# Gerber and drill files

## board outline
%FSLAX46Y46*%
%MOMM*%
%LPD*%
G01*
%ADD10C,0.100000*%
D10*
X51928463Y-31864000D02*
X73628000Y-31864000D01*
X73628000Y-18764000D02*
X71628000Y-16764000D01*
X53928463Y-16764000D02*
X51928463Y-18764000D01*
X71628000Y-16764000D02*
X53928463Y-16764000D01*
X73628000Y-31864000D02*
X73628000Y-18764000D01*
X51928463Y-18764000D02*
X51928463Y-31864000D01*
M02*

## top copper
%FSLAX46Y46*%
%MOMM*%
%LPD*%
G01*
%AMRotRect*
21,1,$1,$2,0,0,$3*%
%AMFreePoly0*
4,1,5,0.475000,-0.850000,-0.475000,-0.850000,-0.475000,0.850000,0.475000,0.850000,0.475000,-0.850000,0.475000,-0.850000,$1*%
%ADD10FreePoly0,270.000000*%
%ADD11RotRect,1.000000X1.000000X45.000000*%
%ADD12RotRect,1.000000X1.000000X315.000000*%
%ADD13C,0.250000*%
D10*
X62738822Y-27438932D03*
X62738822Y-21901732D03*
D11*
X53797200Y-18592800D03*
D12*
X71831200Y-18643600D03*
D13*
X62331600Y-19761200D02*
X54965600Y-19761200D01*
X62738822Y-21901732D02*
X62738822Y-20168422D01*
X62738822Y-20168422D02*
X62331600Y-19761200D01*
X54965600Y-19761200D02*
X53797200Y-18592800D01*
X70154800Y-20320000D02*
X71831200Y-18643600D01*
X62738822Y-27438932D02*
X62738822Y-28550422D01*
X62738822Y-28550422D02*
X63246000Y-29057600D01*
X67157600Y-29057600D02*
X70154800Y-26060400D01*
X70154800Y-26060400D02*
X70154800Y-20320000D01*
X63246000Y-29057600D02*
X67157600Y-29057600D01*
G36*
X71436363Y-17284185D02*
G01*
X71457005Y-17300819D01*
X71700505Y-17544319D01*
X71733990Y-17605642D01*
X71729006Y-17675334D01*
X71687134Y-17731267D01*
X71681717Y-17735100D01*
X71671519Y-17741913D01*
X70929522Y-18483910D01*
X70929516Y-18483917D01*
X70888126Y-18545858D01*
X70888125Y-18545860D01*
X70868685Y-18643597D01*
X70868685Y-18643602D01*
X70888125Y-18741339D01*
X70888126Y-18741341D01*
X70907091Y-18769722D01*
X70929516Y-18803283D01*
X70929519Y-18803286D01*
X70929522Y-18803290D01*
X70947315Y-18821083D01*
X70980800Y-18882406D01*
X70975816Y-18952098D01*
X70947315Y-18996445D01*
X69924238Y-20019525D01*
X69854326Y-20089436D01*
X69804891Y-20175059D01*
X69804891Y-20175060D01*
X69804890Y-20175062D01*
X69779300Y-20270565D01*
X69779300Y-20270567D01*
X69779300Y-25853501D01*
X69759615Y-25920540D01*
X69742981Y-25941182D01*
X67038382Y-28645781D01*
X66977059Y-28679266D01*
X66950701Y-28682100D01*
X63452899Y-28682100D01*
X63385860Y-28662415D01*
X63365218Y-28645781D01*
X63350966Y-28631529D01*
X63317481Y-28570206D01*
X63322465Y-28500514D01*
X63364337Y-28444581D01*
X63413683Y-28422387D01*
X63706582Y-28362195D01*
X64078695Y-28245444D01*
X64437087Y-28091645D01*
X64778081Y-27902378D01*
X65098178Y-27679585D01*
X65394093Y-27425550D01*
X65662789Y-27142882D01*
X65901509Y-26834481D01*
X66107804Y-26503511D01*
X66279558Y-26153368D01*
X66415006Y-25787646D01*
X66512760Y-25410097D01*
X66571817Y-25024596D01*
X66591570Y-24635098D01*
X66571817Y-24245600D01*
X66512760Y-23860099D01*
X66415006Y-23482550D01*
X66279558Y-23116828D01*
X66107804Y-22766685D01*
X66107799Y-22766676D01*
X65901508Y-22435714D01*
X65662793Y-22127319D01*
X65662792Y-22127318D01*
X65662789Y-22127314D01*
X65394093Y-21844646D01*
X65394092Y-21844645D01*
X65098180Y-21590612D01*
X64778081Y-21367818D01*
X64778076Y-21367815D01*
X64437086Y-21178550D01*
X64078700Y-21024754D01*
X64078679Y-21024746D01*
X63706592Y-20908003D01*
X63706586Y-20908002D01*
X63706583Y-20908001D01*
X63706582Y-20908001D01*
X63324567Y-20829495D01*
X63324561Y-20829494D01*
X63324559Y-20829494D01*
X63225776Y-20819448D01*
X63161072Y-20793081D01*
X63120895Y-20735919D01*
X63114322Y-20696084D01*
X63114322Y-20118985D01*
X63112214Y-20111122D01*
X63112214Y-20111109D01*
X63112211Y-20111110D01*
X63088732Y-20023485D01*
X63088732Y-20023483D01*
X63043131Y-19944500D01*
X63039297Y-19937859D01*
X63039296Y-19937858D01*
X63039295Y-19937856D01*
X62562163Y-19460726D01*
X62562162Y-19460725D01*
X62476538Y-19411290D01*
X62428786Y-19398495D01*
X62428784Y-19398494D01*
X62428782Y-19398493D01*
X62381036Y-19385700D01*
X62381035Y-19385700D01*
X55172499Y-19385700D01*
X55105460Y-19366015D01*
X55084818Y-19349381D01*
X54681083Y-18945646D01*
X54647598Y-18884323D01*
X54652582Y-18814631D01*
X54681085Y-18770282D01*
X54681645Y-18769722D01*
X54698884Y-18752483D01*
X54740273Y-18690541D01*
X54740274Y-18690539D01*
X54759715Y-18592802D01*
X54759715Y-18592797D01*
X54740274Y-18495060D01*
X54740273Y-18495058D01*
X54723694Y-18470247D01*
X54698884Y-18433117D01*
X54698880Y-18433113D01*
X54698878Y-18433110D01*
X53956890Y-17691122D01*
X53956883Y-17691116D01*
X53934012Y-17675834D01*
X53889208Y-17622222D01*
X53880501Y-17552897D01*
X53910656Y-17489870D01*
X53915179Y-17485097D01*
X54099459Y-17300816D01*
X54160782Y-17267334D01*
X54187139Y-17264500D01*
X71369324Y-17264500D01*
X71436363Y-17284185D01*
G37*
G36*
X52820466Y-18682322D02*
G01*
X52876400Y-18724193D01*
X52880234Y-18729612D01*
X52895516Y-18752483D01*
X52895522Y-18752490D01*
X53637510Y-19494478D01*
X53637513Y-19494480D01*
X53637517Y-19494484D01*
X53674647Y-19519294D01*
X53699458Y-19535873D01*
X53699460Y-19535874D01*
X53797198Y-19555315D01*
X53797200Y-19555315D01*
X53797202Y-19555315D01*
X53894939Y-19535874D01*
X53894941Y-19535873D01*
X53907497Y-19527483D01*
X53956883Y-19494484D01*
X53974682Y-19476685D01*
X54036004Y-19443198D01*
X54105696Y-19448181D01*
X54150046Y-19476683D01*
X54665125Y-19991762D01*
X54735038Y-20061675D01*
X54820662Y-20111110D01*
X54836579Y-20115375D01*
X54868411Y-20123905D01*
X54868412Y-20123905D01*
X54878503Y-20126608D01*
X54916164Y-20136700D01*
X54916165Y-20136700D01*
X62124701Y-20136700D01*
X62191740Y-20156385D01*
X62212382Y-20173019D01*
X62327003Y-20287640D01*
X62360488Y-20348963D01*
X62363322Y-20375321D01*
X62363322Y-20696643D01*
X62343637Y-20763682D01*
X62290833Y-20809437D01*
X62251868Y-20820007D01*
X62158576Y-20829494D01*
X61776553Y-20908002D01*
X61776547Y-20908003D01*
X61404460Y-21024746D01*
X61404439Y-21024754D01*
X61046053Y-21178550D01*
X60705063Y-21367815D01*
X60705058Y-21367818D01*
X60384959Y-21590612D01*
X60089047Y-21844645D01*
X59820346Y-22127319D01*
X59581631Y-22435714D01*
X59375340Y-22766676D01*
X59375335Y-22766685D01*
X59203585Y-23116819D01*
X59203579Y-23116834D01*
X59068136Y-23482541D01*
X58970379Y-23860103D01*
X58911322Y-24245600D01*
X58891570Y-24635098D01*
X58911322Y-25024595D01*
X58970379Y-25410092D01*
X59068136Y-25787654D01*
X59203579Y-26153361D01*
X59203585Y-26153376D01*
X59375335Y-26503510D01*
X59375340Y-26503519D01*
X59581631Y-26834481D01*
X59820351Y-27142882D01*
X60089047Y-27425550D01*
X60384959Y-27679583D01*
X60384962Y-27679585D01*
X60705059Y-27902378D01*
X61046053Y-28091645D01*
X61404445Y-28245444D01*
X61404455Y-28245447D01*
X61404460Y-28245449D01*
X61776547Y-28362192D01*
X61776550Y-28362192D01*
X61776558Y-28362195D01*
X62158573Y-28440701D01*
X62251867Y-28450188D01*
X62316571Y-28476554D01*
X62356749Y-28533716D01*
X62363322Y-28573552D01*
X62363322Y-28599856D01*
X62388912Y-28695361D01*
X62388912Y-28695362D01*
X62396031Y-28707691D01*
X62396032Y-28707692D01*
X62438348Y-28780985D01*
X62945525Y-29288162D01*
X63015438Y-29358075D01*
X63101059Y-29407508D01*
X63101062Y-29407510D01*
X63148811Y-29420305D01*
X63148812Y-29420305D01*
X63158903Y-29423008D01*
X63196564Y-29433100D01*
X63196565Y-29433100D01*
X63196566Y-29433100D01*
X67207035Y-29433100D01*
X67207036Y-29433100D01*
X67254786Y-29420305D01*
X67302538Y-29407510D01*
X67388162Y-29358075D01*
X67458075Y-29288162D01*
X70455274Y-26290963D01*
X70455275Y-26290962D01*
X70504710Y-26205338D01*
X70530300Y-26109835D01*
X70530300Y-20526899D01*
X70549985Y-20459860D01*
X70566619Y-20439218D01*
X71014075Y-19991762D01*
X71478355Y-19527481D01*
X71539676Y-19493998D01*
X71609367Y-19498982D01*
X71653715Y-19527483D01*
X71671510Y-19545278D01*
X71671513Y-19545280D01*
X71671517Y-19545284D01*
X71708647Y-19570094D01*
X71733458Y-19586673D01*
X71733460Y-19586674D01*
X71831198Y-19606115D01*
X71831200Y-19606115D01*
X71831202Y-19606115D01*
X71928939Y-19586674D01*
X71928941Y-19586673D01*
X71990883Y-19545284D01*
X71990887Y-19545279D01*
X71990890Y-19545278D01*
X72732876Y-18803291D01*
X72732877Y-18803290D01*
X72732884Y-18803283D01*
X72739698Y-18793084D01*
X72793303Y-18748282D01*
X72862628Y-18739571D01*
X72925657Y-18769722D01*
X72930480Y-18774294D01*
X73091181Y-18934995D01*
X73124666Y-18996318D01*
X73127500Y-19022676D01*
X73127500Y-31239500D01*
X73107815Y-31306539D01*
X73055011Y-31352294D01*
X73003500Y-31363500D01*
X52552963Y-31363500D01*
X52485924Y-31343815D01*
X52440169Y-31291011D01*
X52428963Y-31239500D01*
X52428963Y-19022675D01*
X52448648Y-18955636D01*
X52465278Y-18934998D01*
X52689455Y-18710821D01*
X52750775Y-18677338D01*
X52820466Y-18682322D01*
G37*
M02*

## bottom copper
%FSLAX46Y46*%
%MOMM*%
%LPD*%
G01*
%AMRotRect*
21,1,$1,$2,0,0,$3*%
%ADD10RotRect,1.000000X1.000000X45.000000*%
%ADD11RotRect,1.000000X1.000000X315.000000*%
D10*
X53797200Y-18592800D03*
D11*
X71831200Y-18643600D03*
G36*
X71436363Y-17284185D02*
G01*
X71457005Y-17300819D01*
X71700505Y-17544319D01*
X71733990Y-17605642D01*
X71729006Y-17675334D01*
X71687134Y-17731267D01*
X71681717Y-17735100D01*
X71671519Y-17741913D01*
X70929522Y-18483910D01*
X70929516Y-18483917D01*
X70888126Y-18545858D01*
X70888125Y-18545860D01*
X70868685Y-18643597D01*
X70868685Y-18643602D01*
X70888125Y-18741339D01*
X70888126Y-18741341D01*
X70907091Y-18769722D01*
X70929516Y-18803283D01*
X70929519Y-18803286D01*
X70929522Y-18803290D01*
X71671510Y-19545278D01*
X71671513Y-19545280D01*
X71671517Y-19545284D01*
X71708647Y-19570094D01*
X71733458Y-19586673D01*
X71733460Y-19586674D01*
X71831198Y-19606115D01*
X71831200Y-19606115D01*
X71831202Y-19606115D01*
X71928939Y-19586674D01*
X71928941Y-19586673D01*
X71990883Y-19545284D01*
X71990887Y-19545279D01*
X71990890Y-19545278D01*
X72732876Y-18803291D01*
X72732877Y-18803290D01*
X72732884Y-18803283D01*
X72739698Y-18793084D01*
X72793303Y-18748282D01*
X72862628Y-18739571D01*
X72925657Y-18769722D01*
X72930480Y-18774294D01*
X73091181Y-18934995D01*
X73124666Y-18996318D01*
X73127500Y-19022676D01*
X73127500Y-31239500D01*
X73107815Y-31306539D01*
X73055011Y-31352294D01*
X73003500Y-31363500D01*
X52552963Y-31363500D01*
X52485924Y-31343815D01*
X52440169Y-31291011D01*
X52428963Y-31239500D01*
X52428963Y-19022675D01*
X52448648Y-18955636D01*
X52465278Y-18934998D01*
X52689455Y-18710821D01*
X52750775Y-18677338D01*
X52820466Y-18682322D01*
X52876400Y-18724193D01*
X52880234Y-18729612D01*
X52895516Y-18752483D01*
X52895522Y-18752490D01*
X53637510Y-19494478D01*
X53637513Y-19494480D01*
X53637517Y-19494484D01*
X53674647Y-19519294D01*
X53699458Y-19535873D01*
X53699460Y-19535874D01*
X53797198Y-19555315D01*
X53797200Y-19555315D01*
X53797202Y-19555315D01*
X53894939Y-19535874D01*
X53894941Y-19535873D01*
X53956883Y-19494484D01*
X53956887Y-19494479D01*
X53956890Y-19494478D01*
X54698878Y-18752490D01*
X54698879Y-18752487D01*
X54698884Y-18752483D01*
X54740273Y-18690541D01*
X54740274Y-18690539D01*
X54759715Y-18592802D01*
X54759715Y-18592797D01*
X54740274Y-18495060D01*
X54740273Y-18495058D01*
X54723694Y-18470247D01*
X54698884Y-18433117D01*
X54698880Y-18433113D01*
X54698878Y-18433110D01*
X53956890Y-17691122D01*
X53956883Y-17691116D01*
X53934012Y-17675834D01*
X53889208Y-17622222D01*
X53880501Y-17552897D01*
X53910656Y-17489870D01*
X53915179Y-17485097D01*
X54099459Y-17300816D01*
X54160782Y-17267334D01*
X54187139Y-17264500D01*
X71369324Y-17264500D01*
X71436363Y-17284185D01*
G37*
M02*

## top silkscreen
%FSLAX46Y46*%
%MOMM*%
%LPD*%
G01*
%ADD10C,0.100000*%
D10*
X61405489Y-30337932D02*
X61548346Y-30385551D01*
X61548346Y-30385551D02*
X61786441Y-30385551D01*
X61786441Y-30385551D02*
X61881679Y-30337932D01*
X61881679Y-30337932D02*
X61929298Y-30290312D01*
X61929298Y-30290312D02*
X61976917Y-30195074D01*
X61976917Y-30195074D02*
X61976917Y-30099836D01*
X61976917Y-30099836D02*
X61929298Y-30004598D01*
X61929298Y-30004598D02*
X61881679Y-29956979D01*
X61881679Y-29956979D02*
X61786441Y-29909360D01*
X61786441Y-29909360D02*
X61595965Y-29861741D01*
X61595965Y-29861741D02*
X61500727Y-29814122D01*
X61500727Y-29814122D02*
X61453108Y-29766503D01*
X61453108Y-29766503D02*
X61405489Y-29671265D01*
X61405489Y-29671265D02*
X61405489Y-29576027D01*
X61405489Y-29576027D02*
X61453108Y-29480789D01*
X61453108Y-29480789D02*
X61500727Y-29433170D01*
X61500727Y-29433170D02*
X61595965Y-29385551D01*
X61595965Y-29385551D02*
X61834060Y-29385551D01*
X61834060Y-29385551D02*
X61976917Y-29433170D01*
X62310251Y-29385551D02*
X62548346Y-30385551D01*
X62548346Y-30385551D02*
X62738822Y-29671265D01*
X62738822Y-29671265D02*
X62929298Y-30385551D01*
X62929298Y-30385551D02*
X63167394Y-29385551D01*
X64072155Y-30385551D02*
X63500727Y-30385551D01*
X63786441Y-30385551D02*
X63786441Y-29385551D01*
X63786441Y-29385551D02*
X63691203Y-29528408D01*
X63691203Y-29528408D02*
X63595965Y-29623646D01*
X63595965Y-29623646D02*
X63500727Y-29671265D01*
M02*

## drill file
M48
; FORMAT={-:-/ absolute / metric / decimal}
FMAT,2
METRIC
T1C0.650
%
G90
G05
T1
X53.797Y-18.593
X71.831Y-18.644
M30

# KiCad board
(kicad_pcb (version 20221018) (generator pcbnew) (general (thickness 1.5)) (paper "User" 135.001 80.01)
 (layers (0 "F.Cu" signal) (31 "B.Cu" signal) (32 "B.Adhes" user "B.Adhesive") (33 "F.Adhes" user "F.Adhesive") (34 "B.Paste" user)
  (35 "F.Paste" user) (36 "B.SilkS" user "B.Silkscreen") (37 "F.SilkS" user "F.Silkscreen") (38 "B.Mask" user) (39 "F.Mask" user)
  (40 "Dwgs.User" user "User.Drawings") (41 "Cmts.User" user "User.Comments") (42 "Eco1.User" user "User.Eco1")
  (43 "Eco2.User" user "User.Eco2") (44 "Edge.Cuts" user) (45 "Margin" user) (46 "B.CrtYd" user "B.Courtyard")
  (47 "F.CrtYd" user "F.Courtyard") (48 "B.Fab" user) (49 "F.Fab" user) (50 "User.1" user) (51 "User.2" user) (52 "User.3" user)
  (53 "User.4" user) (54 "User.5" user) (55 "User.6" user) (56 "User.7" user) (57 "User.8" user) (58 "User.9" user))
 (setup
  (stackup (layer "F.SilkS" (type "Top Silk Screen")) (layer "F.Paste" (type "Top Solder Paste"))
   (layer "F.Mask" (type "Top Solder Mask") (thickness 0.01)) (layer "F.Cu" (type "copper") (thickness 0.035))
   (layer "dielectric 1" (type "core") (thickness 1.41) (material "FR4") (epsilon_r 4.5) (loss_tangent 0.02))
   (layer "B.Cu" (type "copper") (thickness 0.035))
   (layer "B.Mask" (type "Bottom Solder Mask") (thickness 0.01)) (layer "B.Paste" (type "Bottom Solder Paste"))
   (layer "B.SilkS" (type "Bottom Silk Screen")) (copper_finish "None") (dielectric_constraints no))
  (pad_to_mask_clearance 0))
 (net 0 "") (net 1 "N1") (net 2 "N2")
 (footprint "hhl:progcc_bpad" (layer "F.Cu") (at 62.738822 24.644932)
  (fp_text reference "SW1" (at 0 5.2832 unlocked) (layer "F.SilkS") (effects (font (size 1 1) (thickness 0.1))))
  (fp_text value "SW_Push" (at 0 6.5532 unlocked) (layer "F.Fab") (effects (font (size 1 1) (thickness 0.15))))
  (pad "1" smd custom (at 0 2.794 270) (size 0.95 1.7) (layers "F.Cu") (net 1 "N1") (thermal_bridge_angle 45)
   (options (clearance outline) (anchor rect)) (primitives))
  (pad "2" smd custom (at 0 -2.7432 270) (size 0.95 1.7) (layers "F.Cu") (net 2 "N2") (thermal_bridge_angle 45)
   (options (clearance outline) (anchor rect)) (primitives))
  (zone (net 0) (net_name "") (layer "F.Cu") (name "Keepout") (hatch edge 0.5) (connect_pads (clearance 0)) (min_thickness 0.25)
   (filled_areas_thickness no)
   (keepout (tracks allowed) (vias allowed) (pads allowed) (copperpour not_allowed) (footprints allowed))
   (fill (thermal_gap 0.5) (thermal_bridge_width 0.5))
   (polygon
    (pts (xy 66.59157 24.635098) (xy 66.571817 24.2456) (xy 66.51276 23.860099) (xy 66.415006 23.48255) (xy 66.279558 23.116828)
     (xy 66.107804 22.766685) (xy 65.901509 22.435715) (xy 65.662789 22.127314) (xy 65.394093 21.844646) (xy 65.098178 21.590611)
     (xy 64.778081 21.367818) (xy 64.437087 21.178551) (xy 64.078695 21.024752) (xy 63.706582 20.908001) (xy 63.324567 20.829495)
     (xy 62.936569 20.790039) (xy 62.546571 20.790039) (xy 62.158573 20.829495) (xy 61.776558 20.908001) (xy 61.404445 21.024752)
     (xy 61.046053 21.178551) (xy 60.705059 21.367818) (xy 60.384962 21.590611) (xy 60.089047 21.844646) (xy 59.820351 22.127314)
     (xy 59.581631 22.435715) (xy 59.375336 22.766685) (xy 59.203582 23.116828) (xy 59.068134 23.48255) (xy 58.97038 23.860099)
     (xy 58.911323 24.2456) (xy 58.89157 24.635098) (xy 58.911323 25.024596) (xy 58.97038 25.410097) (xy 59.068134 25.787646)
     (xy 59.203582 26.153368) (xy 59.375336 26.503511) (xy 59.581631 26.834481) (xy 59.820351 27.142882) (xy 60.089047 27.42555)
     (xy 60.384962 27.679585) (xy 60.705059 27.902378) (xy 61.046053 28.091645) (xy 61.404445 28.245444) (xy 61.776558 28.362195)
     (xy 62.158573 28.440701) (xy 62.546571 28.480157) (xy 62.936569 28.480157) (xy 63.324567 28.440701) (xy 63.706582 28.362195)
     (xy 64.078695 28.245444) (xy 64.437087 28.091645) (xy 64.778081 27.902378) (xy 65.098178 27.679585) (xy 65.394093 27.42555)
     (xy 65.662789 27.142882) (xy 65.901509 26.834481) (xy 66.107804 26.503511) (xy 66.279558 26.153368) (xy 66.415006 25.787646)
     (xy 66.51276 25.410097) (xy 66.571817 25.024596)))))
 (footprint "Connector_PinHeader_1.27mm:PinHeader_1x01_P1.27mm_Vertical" (layer "B.Cu") (at 53.7972 18.5928 45)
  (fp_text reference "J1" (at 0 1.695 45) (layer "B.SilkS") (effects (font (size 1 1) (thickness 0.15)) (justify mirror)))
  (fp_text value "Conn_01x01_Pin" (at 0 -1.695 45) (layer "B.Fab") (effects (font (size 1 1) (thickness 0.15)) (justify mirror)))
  (pad "1" thru_hole rect (at 0 0 45) (size 1 1) (drill 0.65) (layers "*.Cu" "*.Mask") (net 2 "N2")))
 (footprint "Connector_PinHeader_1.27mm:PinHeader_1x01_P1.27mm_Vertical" (layer "B.Cu") (at 71.8312 18.6436 -45)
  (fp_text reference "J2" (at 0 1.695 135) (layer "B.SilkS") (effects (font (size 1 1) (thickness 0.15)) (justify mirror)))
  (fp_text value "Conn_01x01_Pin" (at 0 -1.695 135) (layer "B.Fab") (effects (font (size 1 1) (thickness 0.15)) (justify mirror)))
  (pad "1" thru_hole rect (at 0 0 315) (size 1 1) (drill 0.65) (layers "*.Cu" "*.Mask") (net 1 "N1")))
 (gr_line (start 51.928463 31.864) (end 73.628 31.864) (stroke (width 0.1) (type solid)) (layer "Edge.Cuts"))
 (gr_line (start 73.628 18.764) (end 71.628 16.764) (stroke (width 0.1) (type solid)) (layer "Edge.Cuts"))
 (gr_line (start 53.928463 16.764) (end 51.928463 18.764) (stroke (width 0.1) (type solid)) (layer "Edge.Cuts"))
 (gr_line (start 71.628 16.764) (end 53.928463 16.764) (stroke (width 0.1) (type solid)) (layer "Edge.Cuts"))
 (gr_line (start 73.628 31.864) (end 73.628 18.764) (stroke (width 0.1) (type solid)) (layer "Edge.Cuts"))
 (gr_line (start 51.928463 18.764) (end 51.928463 31.864) (stroke (width 0.1) (type solid)) (layer "Edge.Cuts"))
 (segment (start 62.3316 19.7612) (end 54.9656 19.7612) (width 0.25) (layer "F.Cu") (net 2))
 (segment (start 62.738822 21.901732) (end 62.738822 20.168422) (width 0.25) (layer "F.Cu") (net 2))
 (segment (start 62.738822 20.168422) (end 62.3316 19.7612) (width 0.25) (layer "F.Cu") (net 2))
 (segment (start 54.9656 19.7612) (end 53.7972 18.5928) (width 0.25) (layer "F.Cu") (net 2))
 (segment (start 70.1548 20.32) (end 71.8312 18.6436) (width 0.25) (layer "F.Cu") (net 1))
 (segment (start 62.738822 27.438932) (end 62.738822 28.550422) (width 0.25) (layer "F.Cu") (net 1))
 (segment (start 62.738822 28.550422) (end 63.246 29.0576) (width 0.25) (layer "F.Cu") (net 1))
 (segment (start 67.1576 29.0576) (end 70.1548 26.0604) (width 0.25) (layer "F.Cu") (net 1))
 (segment (start 70.1548 26.0604) (end 70.1548 20.32) (width 0.25) (layer "F.Cu") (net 1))
 (segment (start 63.246 29.0576) (end 67.1576 29.0576) (width 0.25) (layer "F.Cu") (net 1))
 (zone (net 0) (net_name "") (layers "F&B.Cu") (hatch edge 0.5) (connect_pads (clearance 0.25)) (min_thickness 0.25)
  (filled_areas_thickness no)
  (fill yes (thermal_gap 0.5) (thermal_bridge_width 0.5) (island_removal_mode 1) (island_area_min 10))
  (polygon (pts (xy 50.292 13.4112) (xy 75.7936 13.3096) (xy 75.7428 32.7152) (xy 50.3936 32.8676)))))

